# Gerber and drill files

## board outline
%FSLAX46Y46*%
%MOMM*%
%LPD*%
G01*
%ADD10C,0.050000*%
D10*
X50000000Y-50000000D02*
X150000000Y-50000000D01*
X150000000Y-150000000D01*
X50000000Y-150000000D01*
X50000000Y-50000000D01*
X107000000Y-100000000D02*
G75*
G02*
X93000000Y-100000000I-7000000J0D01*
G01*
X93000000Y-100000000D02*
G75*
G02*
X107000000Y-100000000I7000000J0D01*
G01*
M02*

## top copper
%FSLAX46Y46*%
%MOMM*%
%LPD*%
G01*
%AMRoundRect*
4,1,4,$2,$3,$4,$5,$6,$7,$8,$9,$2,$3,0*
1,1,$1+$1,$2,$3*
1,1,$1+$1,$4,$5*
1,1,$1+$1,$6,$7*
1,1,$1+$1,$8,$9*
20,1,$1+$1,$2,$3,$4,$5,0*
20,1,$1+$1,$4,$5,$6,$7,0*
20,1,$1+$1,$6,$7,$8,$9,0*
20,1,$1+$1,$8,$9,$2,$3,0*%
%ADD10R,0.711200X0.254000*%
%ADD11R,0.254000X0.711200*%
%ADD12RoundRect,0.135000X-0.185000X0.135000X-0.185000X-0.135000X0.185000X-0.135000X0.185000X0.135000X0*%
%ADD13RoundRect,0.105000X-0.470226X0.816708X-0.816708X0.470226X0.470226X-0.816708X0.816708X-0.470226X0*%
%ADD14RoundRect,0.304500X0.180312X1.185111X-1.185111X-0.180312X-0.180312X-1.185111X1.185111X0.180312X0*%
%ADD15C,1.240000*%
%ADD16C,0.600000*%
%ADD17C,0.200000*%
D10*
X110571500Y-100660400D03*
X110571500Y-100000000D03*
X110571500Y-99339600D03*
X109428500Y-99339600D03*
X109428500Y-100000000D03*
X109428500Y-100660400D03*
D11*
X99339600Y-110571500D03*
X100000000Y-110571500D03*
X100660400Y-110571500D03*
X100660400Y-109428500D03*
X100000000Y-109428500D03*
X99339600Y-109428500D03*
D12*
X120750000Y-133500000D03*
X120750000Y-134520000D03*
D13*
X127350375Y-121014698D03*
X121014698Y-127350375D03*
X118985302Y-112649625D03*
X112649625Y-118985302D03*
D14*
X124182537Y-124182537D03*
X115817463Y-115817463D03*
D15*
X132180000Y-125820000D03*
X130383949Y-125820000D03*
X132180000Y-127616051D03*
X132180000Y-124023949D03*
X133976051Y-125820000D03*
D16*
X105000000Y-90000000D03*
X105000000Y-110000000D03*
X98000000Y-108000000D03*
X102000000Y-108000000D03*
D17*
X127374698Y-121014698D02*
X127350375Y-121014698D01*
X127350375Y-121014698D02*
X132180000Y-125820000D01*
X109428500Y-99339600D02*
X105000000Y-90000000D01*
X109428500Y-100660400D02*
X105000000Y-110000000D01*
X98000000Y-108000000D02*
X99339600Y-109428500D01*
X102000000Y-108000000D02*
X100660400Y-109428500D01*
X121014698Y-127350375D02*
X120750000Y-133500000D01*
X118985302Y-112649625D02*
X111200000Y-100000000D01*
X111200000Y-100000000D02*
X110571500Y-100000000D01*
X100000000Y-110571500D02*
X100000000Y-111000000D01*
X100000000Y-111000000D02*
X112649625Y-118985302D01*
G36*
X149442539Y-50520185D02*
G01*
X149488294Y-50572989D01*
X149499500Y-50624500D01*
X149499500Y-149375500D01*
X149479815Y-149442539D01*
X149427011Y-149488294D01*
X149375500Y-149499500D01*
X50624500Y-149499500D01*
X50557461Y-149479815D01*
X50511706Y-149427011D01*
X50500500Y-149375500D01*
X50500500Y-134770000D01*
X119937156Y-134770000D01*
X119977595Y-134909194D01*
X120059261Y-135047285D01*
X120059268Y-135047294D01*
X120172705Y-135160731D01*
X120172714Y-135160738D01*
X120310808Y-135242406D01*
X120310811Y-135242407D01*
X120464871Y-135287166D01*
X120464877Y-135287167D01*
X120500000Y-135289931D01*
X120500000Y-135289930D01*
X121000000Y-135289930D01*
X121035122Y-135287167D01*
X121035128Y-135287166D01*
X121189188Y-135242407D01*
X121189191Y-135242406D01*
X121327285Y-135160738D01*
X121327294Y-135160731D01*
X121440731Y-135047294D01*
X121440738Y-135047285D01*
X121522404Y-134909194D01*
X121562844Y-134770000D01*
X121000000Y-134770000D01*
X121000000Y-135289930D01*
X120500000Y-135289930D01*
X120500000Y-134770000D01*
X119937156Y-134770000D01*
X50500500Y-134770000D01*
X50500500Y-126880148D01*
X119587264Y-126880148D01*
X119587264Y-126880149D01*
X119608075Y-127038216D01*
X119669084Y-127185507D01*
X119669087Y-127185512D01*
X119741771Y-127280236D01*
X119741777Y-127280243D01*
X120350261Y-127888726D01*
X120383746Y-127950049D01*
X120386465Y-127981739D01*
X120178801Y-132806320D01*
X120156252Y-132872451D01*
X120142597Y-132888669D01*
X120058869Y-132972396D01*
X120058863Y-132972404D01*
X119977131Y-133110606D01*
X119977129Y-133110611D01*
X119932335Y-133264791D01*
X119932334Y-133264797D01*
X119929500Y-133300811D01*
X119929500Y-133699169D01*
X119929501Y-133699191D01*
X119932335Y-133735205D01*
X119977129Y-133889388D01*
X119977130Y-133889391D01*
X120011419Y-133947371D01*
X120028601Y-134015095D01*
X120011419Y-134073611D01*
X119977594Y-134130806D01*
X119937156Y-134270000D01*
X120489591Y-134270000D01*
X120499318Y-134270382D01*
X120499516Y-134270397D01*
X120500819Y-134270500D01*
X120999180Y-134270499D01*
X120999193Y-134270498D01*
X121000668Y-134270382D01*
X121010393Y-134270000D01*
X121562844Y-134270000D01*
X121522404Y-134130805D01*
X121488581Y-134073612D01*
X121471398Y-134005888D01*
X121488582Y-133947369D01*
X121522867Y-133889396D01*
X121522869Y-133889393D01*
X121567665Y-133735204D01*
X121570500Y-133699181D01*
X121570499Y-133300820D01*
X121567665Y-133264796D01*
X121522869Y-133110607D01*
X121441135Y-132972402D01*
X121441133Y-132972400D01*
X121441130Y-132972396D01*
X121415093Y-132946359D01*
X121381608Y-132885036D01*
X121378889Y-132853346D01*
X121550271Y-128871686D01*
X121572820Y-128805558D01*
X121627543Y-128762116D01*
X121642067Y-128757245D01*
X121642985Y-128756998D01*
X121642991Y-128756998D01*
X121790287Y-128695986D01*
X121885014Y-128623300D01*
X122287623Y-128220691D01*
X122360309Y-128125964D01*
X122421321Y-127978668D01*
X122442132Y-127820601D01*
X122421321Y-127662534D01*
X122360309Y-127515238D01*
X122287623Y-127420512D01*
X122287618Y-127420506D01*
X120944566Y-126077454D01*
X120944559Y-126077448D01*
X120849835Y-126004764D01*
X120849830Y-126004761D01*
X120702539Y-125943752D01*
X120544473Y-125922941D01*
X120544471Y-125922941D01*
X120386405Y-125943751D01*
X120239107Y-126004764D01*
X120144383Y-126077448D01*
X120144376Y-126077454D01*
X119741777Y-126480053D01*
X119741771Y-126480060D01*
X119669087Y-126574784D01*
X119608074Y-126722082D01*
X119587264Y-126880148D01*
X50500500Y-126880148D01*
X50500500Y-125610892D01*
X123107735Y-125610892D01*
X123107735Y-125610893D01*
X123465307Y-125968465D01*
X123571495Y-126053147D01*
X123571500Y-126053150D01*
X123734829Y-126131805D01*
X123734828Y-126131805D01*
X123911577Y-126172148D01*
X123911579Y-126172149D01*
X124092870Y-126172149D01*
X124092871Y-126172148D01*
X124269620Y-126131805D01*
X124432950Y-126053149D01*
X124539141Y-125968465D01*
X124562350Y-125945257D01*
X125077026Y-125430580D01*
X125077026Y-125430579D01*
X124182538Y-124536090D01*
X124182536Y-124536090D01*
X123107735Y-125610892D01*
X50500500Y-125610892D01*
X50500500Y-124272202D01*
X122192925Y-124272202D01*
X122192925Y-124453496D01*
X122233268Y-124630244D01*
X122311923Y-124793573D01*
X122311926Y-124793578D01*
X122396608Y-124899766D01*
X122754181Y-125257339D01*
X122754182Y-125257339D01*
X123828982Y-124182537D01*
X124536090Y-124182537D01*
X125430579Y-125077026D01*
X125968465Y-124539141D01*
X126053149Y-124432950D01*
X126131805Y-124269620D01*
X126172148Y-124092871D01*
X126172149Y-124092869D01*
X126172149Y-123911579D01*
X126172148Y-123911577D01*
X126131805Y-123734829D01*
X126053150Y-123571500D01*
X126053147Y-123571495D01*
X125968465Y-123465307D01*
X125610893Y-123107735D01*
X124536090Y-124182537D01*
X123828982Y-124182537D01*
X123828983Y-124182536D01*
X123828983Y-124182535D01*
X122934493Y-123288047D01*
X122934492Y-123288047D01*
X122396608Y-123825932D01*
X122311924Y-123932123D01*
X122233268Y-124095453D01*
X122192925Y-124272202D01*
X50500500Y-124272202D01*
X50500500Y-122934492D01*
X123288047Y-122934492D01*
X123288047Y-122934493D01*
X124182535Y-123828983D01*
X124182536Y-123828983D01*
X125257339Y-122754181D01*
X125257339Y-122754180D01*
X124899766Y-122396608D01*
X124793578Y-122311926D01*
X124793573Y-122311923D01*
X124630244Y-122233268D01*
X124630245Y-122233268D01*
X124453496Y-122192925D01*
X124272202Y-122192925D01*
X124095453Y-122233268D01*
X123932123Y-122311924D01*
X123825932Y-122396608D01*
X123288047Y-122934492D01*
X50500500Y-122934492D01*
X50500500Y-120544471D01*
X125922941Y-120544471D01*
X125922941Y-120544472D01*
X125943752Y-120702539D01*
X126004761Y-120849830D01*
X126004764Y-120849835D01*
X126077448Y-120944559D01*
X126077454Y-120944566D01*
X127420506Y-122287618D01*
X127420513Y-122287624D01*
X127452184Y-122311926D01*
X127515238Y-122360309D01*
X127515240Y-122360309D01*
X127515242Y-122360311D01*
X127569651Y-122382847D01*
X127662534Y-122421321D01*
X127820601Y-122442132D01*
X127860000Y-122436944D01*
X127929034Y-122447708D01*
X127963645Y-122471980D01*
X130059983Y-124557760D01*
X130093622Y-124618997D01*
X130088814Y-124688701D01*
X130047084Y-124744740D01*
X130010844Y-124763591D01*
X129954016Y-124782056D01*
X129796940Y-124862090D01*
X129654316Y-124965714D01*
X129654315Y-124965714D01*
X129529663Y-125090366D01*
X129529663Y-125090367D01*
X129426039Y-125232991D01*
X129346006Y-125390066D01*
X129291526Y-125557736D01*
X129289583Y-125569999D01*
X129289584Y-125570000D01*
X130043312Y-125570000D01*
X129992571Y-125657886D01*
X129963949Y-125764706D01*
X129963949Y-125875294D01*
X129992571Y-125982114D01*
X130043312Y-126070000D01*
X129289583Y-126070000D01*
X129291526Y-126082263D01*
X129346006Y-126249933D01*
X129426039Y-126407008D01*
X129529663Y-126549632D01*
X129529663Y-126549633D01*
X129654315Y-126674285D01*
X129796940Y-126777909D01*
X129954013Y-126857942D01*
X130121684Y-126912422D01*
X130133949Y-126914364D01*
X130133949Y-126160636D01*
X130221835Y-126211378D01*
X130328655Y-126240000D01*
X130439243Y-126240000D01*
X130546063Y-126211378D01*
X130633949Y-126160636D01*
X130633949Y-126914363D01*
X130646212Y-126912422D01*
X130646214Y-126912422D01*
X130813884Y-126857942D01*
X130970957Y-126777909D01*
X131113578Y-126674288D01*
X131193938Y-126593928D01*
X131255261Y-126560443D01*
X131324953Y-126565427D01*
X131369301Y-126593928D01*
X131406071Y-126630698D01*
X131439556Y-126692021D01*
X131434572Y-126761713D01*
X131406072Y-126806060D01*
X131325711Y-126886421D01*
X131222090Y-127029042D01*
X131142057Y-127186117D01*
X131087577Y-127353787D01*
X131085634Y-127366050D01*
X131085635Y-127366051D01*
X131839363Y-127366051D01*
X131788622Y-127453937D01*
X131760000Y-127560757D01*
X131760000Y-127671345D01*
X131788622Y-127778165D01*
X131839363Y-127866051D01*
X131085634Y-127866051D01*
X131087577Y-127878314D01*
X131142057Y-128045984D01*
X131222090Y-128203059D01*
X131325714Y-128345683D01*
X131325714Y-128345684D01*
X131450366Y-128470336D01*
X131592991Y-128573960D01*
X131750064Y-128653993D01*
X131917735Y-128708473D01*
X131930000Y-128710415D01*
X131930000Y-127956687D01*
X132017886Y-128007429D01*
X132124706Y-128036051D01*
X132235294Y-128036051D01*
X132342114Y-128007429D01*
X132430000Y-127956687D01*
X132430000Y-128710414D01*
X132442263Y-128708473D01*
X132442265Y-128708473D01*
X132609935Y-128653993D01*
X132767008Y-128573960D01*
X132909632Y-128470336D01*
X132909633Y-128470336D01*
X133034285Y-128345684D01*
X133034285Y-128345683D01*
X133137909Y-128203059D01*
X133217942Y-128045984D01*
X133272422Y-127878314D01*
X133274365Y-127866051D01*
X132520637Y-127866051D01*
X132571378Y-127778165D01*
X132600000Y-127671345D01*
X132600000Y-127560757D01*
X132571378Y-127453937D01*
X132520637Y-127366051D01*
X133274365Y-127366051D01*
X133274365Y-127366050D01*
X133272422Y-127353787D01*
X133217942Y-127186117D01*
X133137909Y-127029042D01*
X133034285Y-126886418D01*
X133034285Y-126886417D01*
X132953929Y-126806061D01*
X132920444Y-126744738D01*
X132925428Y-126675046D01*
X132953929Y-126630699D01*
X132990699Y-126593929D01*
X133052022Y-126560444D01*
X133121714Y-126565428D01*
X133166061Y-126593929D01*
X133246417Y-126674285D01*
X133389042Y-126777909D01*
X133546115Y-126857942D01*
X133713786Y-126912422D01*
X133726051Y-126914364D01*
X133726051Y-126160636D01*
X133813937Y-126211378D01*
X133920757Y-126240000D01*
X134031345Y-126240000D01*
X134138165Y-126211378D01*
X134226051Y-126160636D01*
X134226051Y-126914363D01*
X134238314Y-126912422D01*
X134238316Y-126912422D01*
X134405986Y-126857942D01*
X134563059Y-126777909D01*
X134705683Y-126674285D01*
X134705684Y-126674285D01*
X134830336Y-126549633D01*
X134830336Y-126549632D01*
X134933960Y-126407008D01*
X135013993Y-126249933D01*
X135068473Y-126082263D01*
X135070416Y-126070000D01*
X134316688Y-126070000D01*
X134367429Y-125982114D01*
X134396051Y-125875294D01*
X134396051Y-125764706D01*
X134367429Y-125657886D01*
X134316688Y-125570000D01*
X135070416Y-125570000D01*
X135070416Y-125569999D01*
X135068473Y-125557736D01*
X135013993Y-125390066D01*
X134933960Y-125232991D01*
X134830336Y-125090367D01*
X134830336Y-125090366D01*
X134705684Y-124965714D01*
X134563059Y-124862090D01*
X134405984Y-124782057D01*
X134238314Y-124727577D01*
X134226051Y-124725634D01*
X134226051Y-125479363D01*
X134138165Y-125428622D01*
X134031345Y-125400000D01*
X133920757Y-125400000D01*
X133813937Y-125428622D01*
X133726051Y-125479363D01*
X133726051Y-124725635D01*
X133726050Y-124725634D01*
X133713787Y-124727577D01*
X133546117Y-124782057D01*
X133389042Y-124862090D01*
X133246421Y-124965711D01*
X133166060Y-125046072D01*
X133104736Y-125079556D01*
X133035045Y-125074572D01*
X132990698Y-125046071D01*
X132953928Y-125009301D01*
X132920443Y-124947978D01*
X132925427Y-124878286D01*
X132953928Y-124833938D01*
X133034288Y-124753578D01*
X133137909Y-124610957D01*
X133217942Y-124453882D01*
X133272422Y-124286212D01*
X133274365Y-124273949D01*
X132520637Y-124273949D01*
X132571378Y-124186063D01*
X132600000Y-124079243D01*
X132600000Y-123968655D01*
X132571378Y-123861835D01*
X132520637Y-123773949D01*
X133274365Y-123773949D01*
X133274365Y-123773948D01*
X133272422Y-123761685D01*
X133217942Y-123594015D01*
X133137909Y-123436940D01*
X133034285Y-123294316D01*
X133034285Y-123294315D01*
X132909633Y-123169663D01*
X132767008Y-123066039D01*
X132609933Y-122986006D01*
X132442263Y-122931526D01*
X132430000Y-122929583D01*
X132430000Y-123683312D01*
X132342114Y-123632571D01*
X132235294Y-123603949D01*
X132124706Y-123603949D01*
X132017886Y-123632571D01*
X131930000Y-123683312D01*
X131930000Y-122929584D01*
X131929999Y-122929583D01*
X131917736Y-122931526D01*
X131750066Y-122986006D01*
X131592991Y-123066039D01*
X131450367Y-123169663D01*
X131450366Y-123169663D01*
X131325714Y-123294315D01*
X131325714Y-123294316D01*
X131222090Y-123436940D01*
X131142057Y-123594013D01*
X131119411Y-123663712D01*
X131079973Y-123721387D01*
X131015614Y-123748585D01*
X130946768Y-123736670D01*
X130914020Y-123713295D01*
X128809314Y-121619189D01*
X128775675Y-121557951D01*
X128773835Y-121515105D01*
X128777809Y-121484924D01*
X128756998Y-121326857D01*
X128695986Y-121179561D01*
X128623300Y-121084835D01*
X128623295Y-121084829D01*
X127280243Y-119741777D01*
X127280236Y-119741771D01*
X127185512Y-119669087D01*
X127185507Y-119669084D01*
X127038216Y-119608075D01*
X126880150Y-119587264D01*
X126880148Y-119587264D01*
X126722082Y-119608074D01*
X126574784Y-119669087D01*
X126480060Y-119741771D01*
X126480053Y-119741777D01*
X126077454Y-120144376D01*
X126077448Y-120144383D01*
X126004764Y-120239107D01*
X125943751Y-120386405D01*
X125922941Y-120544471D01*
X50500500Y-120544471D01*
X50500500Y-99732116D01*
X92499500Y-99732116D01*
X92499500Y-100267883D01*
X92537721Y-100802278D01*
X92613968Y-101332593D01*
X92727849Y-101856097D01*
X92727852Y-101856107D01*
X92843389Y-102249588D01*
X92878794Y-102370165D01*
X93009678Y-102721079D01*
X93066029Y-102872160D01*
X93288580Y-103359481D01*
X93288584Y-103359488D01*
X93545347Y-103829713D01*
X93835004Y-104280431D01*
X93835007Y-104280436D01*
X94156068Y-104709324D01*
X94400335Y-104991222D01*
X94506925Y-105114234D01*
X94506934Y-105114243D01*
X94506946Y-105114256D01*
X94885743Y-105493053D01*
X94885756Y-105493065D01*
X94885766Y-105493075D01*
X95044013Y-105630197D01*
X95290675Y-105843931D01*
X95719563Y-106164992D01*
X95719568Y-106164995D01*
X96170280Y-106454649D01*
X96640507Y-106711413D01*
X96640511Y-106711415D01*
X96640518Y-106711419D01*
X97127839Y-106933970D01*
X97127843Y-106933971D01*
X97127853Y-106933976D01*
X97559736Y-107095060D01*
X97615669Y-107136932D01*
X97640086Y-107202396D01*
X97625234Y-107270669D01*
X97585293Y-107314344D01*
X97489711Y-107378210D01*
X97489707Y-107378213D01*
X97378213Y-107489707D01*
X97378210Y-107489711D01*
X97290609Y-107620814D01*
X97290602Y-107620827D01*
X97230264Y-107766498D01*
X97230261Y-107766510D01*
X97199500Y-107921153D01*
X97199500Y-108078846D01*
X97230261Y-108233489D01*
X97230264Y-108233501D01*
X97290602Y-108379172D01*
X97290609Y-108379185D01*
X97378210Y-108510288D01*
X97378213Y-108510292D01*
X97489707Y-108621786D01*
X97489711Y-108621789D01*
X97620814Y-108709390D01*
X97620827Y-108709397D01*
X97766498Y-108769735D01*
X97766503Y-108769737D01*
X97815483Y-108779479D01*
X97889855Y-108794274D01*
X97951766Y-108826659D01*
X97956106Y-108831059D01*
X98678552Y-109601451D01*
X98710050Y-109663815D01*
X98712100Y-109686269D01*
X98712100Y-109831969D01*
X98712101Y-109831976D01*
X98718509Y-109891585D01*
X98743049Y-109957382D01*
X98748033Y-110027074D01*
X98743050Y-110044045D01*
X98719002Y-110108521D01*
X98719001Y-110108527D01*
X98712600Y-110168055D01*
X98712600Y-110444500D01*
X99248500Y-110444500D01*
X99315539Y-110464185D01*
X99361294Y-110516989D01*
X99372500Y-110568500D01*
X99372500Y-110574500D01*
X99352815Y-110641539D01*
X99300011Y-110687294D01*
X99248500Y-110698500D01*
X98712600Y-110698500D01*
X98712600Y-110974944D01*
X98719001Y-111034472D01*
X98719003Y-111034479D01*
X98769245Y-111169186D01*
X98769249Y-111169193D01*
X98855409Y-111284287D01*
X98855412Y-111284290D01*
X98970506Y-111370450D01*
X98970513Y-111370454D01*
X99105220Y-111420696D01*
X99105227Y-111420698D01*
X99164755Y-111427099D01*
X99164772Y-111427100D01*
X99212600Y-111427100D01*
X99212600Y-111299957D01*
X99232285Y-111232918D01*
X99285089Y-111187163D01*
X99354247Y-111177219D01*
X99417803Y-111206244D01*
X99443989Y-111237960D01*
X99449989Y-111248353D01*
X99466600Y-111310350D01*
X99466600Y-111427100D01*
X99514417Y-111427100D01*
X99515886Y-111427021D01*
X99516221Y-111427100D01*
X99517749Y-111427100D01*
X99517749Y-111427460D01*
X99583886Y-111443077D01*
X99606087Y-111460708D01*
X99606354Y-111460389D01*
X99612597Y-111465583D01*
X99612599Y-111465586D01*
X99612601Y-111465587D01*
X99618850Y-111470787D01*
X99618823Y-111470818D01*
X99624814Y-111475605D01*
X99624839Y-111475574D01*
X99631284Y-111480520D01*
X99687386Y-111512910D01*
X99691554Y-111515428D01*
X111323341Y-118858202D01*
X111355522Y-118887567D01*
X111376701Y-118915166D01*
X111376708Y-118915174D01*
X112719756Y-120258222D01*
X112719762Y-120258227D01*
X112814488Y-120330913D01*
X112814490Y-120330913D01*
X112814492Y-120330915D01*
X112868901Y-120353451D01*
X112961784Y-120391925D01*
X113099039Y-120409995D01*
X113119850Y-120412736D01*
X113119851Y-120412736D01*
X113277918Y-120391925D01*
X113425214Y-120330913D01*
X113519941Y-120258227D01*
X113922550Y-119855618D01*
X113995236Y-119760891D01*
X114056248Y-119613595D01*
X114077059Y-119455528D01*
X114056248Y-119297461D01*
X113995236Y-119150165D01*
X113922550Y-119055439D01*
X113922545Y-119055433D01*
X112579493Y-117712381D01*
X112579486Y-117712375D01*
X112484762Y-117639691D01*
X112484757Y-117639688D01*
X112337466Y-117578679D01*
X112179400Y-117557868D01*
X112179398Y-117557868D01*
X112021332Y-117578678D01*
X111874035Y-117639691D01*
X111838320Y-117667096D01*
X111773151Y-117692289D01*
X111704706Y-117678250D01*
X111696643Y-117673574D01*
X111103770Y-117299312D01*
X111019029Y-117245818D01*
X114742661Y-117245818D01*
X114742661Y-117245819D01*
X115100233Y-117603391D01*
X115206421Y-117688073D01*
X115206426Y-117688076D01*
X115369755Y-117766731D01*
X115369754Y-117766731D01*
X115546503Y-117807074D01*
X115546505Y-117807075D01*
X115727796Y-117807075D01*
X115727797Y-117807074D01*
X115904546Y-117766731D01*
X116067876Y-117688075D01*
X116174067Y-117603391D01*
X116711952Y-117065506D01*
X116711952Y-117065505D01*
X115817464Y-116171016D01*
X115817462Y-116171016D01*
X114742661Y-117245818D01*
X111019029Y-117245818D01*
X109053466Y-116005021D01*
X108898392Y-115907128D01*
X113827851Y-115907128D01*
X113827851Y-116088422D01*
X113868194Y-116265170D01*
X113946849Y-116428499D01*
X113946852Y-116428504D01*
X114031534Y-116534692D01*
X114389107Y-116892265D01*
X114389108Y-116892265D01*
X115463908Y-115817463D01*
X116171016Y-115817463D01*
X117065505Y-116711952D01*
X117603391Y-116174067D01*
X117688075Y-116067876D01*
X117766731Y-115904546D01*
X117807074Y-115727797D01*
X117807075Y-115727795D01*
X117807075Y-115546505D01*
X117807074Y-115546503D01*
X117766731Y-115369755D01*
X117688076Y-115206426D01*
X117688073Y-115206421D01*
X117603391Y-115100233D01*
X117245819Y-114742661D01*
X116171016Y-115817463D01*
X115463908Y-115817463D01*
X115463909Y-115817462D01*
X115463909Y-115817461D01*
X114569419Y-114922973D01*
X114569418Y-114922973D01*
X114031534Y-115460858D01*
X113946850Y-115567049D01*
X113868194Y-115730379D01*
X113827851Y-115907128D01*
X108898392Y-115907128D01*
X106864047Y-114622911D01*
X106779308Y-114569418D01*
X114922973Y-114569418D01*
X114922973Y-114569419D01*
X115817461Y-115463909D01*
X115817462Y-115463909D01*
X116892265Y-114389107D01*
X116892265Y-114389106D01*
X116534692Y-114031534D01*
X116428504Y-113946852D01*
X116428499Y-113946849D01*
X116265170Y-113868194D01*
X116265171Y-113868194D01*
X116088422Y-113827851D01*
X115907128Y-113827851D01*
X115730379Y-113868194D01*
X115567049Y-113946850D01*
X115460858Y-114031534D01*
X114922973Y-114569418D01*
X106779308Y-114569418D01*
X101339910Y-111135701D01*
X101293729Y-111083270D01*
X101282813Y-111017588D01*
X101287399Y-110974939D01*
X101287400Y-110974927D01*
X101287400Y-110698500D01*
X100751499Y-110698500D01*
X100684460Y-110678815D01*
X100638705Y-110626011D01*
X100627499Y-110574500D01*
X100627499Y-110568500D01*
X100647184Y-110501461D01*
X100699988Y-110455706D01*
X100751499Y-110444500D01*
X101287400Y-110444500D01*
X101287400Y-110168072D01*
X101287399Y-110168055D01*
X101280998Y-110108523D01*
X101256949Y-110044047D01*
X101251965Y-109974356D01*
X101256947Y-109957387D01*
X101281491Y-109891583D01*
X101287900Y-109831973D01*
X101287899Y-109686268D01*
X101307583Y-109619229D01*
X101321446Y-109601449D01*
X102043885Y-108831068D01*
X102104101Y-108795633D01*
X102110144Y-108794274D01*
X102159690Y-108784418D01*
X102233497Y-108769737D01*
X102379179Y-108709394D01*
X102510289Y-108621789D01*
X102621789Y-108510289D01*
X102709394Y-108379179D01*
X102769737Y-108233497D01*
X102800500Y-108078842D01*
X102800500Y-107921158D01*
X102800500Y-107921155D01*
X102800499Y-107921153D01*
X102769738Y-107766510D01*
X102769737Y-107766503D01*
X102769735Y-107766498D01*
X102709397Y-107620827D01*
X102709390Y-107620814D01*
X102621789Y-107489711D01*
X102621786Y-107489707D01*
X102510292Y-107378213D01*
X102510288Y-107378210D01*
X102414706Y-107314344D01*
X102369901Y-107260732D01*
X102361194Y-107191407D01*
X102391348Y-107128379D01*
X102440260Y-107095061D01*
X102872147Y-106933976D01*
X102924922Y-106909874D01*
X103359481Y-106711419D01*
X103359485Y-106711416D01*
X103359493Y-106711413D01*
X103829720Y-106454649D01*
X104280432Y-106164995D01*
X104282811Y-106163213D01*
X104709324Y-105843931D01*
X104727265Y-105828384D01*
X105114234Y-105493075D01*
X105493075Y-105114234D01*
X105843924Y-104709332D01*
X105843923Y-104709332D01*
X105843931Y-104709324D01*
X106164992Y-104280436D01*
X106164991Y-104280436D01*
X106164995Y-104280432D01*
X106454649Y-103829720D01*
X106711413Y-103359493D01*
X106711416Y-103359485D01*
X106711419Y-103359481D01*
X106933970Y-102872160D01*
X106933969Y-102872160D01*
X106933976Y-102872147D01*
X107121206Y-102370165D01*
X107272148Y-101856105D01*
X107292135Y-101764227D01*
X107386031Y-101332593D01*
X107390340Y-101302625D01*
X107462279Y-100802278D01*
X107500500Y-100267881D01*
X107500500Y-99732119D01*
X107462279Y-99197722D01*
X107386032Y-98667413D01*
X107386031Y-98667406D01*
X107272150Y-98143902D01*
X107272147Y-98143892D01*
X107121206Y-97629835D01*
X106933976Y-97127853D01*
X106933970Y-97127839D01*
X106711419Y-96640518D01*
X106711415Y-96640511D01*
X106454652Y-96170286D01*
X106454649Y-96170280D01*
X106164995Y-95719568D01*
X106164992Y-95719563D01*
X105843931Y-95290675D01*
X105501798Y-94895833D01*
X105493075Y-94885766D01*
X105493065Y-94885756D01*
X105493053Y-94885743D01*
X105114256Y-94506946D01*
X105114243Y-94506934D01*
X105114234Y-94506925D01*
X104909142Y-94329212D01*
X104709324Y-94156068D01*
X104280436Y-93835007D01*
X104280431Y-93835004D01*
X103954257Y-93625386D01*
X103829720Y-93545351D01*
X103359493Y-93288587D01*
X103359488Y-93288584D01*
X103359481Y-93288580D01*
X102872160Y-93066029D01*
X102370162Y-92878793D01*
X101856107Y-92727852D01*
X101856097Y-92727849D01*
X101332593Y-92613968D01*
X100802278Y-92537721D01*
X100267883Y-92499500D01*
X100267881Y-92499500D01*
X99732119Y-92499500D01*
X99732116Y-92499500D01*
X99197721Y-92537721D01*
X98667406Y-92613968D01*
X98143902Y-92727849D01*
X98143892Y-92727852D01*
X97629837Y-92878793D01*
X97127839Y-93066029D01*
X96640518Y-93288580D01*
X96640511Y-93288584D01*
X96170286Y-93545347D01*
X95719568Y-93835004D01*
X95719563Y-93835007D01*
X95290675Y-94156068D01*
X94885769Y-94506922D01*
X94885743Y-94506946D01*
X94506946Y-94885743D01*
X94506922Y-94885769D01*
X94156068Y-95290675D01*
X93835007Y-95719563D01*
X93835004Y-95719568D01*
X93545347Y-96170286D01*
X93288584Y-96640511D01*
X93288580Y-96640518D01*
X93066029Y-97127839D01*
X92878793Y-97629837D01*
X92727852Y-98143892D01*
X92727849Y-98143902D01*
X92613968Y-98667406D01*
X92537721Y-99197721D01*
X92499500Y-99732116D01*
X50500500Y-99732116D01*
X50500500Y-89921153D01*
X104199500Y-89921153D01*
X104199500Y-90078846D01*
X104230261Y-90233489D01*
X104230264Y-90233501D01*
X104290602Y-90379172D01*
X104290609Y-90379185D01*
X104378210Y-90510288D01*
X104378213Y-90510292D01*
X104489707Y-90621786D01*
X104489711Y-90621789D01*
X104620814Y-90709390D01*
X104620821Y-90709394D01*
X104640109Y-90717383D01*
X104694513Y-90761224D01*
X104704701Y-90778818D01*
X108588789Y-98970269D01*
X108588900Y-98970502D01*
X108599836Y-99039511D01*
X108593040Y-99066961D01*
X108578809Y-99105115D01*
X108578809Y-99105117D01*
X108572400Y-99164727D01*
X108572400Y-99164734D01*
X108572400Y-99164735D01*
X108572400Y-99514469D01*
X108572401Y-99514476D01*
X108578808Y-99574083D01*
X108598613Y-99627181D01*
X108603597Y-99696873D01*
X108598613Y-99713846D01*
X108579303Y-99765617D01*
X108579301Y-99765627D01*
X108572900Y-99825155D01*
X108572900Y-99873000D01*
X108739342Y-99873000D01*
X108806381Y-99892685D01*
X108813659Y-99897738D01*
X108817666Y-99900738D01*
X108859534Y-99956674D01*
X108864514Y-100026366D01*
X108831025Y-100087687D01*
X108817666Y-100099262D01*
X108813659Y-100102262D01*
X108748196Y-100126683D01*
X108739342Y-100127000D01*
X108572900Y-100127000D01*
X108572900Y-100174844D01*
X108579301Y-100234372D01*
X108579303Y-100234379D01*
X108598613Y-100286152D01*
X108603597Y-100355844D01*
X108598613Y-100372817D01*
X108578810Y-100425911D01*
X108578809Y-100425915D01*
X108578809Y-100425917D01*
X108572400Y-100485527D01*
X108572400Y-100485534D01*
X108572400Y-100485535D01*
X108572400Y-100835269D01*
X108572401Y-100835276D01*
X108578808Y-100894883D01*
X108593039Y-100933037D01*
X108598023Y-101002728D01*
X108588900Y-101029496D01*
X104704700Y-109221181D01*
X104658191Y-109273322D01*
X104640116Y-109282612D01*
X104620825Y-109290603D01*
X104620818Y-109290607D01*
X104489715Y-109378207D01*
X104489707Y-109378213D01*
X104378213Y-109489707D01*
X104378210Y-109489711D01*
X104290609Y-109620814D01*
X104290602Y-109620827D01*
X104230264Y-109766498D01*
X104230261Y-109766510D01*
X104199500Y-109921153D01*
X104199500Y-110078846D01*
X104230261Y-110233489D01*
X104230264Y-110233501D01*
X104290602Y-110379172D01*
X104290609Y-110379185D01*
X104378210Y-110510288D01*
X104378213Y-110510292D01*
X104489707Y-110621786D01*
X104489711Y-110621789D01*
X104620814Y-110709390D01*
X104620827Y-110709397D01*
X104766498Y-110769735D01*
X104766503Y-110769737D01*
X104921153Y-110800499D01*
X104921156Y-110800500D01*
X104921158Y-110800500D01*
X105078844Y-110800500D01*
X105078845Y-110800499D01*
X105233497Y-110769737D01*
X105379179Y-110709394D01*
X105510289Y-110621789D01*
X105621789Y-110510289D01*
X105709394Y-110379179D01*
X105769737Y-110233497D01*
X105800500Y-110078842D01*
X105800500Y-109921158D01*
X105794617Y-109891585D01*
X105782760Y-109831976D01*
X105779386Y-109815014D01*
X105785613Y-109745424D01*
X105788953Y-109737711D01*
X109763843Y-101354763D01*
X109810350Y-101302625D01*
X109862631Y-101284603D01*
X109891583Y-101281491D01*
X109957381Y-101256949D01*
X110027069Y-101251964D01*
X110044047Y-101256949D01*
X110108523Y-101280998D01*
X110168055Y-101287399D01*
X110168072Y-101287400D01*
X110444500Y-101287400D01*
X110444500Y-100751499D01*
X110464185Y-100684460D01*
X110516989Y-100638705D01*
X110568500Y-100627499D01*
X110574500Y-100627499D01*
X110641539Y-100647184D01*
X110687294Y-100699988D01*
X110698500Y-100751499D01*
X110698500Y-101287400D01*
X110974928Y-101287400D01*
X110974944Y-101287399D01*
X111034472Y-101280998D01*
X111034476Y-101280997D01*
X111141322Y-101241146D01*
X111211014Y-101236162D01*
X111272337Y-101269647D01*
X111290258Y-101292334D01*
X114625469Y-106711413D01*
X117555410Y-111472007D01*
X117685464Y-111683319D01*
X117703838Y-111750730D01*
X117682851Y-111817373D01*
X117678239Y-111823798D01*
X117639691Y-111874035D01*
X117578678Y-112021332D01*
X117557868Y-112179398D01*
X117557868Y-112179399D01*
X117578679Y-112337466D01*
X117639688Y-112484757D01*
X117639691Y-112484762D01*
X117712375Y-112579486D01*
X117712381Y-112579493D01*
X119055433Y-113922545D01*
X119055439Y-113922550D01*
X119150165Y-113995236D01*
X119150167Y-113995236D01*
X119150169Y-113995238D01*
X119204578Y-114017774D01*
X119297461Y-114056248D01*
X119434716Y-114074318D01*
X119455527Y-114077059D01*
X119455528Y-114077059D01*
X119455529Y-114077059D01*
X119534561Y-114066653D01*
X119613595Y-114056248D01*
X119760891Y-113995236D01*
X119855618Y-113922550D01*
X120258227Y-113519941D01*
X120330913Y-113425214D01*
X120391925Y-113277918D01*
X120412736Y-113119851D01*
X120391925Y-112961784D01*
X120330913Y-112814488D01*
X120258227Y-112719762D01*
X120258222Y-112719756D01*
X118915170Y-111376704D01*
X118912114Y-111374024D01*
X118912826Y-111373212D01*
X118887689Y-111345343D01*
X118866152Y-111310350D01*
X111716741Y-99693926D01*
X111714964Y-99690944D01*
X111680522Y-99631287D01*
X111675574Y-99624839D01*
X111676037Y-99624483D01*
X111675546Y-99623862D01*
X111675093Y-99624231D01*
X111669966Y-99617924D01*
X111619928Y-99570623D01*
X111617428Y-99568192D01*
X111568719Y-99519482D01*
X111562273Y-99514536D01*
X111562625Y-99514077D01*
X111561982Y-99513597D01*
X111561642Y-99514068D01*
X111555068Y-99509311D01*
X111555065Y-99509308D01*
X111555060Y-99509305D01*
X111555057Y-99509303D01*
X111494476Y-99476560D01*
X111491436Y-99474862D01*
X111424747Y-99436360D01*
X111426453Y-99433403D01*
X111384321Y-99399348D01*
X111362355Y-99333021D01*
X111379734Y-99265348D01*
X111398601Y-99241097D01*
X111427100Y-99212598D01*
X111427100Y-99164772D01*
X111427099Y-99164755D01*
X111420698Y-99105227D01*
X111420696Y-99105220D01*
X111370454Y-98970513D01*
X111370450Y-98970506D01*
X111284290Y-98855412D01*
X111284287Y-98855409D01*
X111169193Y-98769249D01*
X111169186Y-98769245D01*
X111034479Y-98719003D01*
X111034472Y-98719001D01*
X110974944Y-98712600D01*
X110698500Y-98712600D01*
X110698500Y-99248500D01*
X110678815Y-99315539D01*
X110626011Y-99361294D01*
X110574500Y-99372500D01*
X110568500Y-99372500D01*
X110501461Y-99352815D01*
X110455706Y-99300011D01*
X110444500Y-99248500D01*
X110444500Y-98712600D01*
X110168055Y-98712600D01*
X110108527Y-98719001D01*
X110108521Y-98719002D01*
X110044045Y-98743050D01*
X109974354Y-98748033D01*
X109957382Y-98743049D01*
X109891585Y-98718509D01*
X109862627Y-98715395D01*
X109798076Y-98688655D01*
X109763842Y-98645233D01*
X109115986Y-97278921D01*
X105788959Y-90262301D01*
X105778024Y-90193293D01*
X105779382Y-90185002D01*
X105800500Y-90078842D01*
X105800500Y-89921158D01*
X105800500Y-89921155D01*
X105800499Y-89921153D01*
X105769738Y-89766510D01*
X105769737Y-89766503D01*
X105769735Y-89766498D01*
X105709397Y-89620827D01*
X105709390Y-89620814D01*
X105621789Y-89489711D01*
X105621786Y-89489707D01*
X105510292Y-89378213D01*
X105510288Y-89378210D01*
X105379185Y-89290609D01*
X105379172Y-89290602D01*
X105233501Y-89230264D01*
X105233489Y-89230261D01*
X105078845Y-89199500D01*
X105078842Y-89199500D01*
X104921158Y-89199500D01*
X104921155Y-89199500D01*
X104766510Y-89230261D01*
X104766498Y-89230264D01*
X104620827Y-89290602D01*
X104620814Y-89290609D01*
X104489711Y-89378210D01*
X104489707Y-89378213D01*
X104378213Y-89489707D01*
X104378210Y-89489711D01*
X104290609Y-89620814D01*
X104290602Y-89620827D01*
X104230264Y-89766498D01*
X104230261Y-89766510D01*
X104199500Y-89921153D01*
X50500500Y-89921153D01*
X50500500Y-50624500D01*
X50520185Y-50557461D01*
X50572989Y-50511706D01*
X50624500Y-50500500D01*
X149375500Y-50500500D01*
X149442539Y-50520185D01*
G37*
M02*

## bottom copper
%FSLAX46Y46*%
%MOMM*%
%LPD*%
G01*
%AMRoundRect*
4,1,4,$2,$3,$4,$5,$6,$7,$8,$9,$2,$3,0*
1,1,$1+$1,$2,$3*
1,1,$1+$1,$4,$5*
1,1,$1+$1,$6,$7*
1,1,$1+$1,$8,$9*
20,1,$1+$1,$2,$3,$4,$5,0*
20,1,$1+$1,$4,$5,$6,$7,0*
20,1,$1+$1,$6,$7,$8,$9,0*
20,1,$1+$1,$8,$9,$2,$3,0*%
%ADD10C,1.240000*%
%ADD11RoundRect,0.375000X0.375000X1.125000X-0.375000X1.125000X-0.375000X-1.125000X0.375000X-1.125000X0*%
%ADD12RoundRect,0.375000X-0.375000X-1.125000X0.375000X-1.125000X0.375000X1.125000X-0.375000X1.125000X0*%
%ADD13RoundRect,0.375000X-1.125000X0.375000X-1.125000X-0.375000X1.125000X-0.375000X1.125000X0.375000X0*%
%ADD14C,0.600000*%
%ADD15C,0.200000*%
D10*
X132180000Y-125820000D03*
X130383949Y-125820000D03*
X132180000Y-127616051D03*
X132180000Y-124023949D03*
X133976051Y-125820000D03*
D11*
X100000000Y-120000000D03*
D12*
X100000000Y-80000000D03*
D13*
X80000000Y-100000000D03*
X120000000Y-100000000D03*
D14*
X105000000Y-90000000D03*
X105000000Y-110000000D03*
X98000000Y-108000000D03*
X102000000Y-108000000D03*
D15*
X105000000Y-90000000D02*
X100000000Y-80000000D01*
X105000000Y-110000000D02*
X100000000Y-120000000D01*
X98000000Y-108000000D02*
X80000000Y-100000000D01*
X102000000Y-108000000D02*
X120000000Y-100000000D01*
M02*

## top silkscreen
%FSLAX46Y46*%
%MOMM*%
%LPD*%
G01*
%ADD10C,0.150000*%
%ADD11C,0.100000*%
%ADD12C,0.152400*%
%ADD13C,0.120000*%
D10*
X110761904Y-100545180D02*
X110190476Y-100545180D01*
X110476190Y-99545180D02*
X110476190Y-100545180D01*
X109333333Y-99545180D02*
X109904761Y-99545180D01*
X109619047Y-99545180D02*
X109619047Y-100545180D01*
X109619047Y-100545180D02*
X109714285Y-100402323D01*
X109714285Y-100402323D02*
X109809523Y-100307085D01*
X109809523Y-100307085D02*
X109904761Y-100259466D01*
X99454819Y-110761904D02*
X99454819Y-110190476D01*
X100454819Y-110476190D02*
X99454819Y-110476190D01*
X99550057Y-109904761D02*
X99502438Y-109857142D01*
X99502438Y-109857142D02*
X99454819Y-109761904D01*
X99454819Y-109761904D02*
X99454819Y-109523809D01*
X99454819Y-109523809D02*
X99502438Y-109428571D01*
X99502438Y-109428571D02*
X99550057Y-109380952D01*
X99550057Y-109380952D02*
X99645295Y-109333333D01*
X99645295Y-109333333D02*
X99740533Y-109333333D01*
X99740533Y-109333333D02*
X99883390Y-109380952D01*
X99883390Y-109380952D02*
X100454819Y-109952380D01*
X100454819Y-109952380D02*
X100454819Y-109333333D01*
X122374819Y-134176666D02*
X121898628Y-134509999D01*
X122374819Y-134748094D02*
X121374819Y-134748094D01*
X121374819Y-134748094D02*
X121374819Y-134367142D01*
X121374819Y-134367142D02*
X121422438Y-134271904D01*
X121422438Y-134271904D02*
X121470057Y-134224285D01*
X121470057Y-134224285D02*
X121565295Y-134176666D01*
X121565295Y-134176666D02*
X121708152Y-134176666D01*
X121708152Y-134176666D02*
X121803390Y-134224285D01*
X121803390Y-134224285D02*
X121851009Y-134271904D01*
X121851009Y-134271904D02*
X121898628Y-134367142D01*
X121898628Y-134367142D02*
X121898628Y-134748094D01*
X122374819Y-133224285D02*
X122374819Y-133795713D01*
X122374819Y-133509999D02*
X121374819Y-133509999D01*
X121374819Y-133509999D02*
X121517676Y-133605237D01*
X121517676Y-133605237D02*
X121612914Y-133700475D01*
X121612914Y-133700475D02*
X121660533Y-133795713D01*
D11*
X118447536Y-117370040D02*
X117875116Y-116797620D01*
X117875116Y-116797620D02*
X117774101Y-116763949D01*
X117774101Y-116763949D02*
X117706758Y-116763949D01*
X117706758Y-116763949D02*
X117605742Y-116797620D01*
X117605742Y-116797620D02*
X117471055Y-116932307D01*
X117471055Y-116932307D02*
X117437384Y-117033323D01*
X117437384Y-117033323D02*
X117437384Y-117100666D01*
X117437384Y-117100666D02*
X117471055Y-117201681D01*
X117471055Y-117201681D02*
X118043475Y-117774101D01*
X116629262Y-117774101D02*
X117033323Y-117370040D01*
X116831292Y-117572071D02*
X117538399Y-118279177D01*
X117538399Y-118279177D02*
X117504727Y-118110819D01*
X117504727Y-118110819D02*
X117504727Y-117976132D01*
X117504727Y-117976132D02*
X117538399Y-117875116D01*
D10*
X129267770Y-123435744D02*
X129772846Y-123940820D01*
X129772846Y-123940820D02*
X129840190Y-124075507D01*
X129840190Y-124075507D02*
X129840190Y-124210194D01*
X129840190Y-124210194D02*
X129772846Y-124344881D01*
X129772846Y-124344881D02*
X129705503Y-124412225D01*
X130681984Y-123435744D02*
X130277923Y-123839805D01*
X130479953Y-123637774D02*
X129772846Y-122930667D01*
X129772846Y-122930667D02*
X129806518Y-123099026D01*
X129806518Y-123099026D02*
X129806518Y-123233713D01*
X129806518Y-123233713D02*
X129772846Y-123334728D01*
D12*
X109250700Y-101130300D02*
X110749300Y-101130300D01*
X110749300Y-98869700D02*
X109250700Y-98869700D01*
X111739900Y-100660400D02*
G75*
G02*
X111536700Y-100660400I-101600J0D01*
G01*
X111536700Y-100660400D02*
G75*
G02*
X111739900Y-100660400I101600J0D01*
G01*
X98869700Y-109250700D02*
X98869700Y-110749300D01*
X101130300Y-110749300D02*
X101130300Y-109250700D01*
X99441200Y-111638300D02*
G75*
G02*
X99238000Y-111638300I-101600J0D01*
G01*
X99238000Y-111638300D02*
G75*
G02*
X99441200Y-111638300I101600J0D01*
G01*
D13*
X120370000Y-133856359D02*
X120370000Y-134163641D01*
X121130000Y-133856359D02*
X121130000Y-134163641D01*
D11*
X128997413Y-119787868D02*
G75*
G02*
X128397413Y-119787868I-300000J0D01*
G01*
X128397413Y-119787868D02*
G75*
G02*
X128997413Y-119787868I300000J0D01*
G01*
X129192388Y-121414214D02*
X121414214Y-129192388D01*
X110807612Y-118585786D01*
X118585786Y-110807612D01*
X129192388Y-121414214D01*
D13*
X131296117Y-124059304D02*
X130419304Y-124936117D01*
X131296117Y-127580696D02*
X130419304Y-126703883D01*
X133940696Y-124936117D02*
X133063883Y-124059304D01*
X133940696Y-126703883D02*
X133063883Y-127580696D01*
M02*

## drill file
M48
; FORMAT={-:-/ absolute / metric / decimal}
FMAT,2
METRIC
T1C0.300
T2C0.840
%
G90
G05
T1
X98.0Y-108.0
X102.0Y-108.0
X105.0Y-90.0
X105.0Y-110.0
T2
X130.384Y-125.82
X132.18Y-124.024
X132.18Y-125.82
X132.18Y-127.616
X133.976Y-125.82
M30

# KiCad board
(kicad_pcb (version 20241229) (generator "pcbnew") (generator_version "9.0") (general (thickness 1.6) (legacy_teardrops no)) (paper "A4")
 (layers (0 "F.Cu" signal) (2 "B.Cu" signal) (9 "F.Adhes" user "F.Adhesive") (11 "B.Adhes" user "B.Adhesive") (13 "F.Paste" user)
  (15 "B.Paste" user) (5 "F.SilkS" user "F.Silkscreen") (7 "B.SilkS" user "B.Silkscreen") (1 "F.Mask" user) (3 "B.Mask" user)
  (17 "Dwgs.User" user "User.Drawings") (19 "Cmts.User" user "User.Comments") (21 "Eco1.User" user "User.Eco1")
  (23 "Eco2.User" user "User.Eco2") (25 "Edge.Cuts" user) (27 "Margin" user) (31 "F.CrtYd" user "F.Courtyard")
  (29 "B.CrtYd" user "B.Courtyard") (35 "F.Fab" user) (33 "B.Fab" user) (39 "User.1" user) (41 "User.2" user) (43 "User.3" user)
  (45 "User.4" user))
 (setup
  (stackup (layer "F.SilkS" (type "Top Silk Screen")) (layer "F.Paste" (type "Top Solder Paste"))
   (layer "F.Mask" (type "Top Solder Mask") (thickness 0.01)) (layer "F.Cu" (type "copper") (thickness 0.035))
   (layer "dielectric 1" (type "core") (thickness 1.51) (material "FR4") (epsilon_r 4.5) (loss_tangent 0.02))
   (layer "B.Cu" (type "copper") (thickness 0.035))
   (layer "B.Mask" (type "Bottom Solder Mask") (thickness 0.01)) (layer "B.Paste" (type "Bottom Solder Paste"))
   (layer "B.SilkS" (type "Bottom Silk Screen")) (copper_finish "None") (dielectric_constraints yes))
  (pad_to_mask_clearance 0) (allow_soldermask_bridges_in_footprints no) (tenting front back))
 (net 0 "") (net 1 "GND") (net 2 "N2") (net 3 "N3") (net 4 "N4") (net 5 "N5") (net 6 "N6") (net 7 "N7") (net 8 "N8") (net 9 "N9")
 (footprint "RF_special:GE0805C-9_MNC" (layer "F.Cu") (at 110 100 180)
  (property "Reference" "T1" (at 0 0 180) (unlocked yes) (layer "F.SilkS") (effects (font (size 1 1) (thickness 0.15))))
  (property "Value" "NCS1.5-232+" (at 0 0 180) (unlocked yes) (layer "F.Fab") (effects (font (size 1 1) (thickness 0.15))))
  (fp_line (start 0.7493 -1.1303) (end -0.7493 -1.1303) (stroke (width 0.1524) (type solid)) (layer "F.SilkS"))
  (fp_line (start -0.7493 1.1303) (end 0.7493 1.1303) (stroke (width 0.1524) (type solid)) (layer "F.SilkS"))
  (fp_circle (center -1.6383 -0.6604) (end -1.5367 -0.6604) (stroke (width 0.1524) (type solid)) (fill no) (layer "F.SilkS"))
  (pad "1" smd rect (at -0.5715 -0.6604 180) (size 0.7112 0.254) (layers "F.Cu" "F.Mask" "F.Paste") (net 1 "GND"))
  (pad "2" smd rect (at -0.5715 0 180) (size 0.7112 0.254) (layers "F.Cu" "F.Mask" "F.Paste") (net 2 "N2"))
  (pad "3" smd rect (at -0.5715 0.6604 180) (size 0.7112 0.254) (layers "F.Cu" "F.Mask" "F.Paste") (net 1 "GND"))
  (pad "4" smd rect (at 0.5715 0.6604 180) (size 0.7112 0.254) (layers "F.Cu" "F.Mask" "F.Paste") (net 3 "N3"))
  (pad "5" smd rect (at 0.5715 0 180) (size 0.7112 0.254) (layers "F.Cu" "F.Mask" "F.Paste") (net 1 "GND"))
  (pad "6" smd rect (at 0.5715 -0.6604 180) (size 0.7112 0.254) (layers "F.Cu" "F.Mask" "F.Paste") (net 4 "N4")))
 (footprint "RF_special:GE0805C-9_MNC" (layer "F.Cu") (at 100 110 90)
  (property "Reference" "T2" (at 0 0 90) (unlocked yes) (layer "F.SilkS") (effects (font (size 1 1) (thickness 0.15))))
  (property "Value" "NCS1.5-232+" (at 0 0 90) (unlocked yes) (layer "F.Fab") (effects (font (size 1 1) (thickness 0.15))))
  (fp_line (start 0.7493 -1.1303) (end -0.7493 -1.1303) (stroke (width 0.1524) (type solid)) (layer "F.SilkS"))
  (fp_line (start -0.7493 1.1303) (end 0.7493 1.1303) (stroke (width 0.1524) (type solid)) (layer "F.SilkS"))
  (fp_circle (center -1.6383 -0.6604) (end -1.5367 -0.6604) (stroke (width 0.1524) (type solid)) (fill no) (layer "F.SilkS"))
  (pad "1" smd rect (at -0.5715 -0.6604 90) (size 0.7112 0.254) (layers "F.Cu" "F.Mask" "F.Paste") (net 1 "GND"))
  (pad "2" smd rect (at -0.5715 0 90) (size 0.7112 0.254) (layers "F.Cu" "F.Mask" "F.Paste") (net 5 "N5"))
  (pad "3" smd rect (at -0.5715 0.6604 90) (size 0.7112 0.254) (layers "F.Cu" "F.Mask" "F.Paste") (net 1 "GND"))
  (pad "4" smd rect (at 0.5715 0.6604 90) (size 0.7112 0.254) (layers "F.Cu" "F.Mask" "F.Paste") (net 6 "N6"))
  (pad "5" smd rect (at 0.5715 0 90) (size 0.7112 0.254) (layers "F.Cu" "F.Mask" "F.Paste") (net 1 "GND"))
  (pad "6" smd rect (at 0.5715 -0.6604 90) (size 0.7112 0.254) (layers "F.Cu" "F.Mask" "F.Paste") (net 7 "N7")))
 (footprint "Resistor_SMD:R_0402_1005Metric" (layer "F.Cu") (at 120.75 134.01 -90)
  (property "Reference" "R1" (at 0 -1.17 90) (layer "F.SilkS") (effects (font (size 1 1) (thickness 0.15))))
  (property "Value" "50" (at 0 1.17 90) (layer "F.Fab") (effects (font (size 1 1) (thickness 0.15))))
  (fp_line (start -0.153641 0.38) (end 0.153641 0.38) (stroke (width 0.12) (type solid)) (layer "F.SilkS"))
  (fp_line (start -0.153641 -0.38) (end 0.153641 -0.38) (stroke (width 0.12) (type solid)) (layer "F.SilkS"))
  (pad "1" smd roundrect (at -0.51 0 270) (size 0.54 0.64) (layers "F.Cu" "F.Mask" "F.Paste") (roundrect_rratio 0.25) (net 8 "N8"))
  (pad "2" smd roundrect (at 0.51 0 270) (size 0.54 0.64) (layers "F.Cu" "F.Mask" "F.Paste") (roundrect_rratio 0.25) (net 1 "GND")))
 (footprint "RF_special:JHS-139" (layer "F.Cu") (at 120 120 -135)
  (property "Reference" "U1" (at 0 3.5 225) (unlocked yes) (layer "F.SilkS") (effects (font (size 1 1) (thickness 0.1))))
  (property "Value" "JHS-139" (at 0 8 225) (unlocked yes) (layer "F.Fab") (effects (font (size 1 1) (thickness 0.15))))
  (fp_circle (center -6.3 -6) (end -6 -6) (stroke (width 0.1) (type solid)) (fill no) (layer "F.SilkS"))
  (fp_poly (pts (xy -5.5 -7.5) (xy 5.5 -7.5) (xy 5.5 7.5) (xy -5.5 7.5)) (stroke (width 0.1) (type default)) (fill no) (layer "F.SilkS"))
  (pad "1" smd roundrect (at -4.48 -5.915 225) (size 0.7 2.03) (layers "F.Cu" "F.Mask" "F.Paste") (roundrect_rratio 0.15) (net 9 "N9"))
  (pad "2" smd roundrect (at 4.48 -5.915 225) (size 0.7 2.03) (layers "F.Cu" "F.Mask" "F.Paste") (roundrect_rratio 0.15) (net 8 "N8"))
  (pad "3" smd roundrect (at -4.48 5.915 225) (size 0.7 2.03) (layers "F.Cu" "F.Mask" "F.Paste") (roundrect_rratio 0.15) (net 2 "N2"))
  (pad "4" smd roundrect (at 4.48 5.915 225) (size 0.7 2.03) (layers "F.Cu" "F.Mask" "F.Paste") (roundrect_rratio 0.15) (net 5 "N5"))
  (pad "GND" smd roundrect (at 0 -5.915001 225) (size 2.54 2.03) (layers "F.Cu" "F.Mask" "F.Paste") (roundrect_rratio 0.15) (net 1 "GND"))
  (pad "GND" smd roundrect (at 0 5.915001 225) (size 2.54 2.03) (layers "F.Cu" "F.Mask" "F.Paste") (roundrect_rratio 0.15) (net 1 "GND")))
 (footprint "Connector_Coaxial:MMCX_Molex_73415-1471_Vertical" (layer "F.Cu") (at 132.18 125.82 45)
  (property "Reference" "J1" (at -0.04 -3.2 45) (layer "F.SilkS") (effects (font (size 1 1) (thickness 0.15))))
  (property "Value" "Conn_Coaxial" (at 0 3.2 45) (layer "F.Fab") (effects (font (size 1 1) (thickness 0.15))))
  (fp_line (start 0.62 -1.87) (end -0.62 -1.87) (stroke (width 0.12) (type solid)) (layer "F.SilkS"))
  (fp_line (start -1.87 0.62) (end -1.87 -0.62) (stroke (width 0.12) (type solid)) (layer "F.SilkS"))
  (fp_line (start 1.87 0.62) (end 1.87 -0.62) (stroke (width 0.12) (type solid)) (layer "F.SilkS"))
  (fp_line (start 0.62 1.87) (end -0.62 1.87) (stroke (width 0.12) (type solid)) (layer "F.SilkS"))
  (pad "1" thru_hole circle (at 0 0 45) (size 1.24 1.24) (drill 0.84) (layers "*.Cu" "*.Mask") (remove_unused_layers no) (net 9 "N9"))
  (pad "2" thru_hole circle (at -1.27 -1.27 45) (size 1.24 1.24) (drill 0.84) (layers "*.Cu" "*.Mask") (remove_unused_layers no)
   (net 1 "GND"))
  (pad "2" thru_hole circle (at -1.27 1.27 45) (size 1.24 1.24) (drill 0.84) (layers "*.Cu" "*.Mask") (remove_unused_layers no)
   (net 1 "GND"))
  (pad "2" thru_hole circle (at 1.27 -1.27 45) (size 1.24 1.24) (drill 0.84) (layers "*.Cu" "*.Mask") (remove_unused_layers no)
   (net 1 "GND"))
  (pad "2" thru_hole circle (at 1.27 1.27 45) (size 1.24 1.24) (drill 0.84) (layers "*.Cu" "*.Mask") (remove_unused_layers no) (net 1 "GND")))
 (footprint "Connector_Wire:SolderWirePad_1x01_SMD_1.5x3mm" (layer "B.Cu") (at 100 120 180)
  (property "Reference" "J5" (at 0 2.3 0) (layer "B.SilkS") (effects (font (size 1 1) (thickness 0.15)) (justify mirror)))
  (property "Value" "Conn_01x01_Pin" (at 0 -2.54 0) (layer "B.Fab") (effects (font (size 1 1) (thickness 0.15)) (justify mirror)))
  (pad "1" smd roundrect (at 0 0 180) (size 1.5 3) (layers "B.Cu" "B.Mask") (roundrect_rratio 0.25) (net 4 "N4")))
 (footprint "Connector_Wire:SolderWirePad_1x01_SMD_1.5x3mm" (layer "B.Cu") (at 100 80)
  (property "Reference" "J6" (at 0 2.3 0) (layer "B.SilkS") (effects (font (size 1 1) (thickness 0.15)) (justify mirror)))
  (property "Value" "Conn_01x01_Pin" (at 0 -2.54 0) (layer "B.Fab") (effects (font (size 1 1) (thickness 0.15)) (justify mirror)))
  (pad "1" smd roundrect (at 0 0) (size 1.5 3) (layers "B.Cu" "B.Mask") (roundrect_rratio 0.25) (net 3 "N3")))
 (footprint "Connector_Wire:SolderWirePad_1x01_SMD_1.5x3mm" (layer "B.Cu") (at 80 100 -90)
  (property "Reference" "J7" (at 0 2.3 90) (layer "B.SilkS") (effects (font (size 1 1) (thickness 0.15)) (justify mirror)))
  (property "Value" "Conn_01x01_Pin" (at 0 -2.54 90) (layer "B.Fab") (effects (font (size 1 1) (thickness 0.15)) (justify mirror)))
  (pad "1" smd roundrect (at 0 0 270) (size 1.5 3) (layers "B.Cu" "B.Mask") (roundrect_rratio 0.25) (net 7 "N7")))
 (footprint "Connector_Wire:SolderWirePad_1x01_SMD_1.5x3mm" (layer "B.Cu") (at 120 100 -90)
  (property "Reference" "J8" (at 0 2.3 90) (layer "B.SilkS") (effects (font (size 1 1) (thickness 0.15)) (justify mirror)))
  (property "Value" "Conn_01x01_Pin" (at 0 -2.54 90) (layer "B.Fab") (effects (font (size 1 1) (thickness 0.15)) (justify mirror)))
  (pad "1" smd roundrect (at 0 0 270) (size 1.5 3) (layers "B.Cu" "B.Mask") (roundrect_rratio 0.25) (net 6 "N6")))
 (gr_rect (start 50 50) (end 150 150) (stroke (width 0.05) (type solid)) (fill no) (layer "Edge.Cuts"))
 (gr_circle (center 100 100) (end 107 100) (stroke (width 0.05) (type solid)) (fill no) (layer "Edge.Cuts"))
 (segment (start 127.374698 121.014698) (end 127.350375 121.014698) (width 0.2) (layer "F.Cu") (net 9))
 (segment (start 127.350375 121.014698) (end 132.18 125.82) (width 0.2) (layer "F.Cu") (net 9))
 (segment (start 109.4285 99.3396) (end 105 90) (width 0.2) (layer "F.Cu") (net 3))
 (via (at 105 90) (size 0.6) (drill 0.3) (layers "F.Cu" "B.Cu") (free yes) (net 3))
 (segment (start 105 90) (end 100 80) (width 0.2) (layer "B.Cu") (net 3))
 (segment (start 109.4285 100.6604) (end 105 110) (width 0.2) (layer "F.Cu") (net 4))
 (via (at 105 110) (size 0.6) (drill 0.3) (layers "F.Cu" "B.Cu") (free yes) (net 4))
 (segment (start 105 110) (end 100 120) (width 0.2) (layer "B.Cu") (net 4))
 (segment (start 98 108) (end 99.3396 109.4285) (width 0.2) (layer "F.Cu") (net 7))
 (via (at 98 108) (size 0.6) (drill 0.3) (layers "F.Cu" "B.Cu") (free yes) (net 7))
 (segment (start 98 108) (end 80 100) (width 0.2) (layer "B.Cu") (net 7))
 (segment (start 102 108) (end 100.6604 109.4285) (width 0.2) (layer "F.Cu") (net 6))
 (via (at 102 108) (size 0.6) (drill 0.3) (layers "F.Cu" "B.Cu") (free yes) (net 6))
 (segment (start 102 108) (end 120 100) (width 0.2) (layer "B.Cu") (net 6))
 (segment (start 121.014698 127.350375) (end 120.75 133.5) (width 0.2) (layer "F.Cu") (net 8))
 (segment (start 118.985302 112.649625) (end 111.2 100) (width 0.2) (layer "F.Cu") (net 2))
 (segment (start 111.2 100) (end 110.5715 100) (width 0.2) (layer "F.Cu") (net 2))
 (segment (start 100 110.5715) (end 100 111) (width 0.2) (layer "F.Cu") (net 5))
 (segment (start 100 111) (end 112.649625 118.985302) (width 0.2) (layer "F.Cu") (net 5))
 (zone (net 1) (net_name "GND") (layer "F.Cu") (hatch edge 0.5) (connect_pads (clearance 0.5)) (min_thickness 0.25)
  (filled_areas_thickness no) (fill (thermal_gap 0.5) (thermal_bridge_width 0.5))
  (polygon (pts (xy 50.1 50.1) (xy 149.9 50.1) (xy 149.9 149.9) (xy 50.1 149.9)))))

